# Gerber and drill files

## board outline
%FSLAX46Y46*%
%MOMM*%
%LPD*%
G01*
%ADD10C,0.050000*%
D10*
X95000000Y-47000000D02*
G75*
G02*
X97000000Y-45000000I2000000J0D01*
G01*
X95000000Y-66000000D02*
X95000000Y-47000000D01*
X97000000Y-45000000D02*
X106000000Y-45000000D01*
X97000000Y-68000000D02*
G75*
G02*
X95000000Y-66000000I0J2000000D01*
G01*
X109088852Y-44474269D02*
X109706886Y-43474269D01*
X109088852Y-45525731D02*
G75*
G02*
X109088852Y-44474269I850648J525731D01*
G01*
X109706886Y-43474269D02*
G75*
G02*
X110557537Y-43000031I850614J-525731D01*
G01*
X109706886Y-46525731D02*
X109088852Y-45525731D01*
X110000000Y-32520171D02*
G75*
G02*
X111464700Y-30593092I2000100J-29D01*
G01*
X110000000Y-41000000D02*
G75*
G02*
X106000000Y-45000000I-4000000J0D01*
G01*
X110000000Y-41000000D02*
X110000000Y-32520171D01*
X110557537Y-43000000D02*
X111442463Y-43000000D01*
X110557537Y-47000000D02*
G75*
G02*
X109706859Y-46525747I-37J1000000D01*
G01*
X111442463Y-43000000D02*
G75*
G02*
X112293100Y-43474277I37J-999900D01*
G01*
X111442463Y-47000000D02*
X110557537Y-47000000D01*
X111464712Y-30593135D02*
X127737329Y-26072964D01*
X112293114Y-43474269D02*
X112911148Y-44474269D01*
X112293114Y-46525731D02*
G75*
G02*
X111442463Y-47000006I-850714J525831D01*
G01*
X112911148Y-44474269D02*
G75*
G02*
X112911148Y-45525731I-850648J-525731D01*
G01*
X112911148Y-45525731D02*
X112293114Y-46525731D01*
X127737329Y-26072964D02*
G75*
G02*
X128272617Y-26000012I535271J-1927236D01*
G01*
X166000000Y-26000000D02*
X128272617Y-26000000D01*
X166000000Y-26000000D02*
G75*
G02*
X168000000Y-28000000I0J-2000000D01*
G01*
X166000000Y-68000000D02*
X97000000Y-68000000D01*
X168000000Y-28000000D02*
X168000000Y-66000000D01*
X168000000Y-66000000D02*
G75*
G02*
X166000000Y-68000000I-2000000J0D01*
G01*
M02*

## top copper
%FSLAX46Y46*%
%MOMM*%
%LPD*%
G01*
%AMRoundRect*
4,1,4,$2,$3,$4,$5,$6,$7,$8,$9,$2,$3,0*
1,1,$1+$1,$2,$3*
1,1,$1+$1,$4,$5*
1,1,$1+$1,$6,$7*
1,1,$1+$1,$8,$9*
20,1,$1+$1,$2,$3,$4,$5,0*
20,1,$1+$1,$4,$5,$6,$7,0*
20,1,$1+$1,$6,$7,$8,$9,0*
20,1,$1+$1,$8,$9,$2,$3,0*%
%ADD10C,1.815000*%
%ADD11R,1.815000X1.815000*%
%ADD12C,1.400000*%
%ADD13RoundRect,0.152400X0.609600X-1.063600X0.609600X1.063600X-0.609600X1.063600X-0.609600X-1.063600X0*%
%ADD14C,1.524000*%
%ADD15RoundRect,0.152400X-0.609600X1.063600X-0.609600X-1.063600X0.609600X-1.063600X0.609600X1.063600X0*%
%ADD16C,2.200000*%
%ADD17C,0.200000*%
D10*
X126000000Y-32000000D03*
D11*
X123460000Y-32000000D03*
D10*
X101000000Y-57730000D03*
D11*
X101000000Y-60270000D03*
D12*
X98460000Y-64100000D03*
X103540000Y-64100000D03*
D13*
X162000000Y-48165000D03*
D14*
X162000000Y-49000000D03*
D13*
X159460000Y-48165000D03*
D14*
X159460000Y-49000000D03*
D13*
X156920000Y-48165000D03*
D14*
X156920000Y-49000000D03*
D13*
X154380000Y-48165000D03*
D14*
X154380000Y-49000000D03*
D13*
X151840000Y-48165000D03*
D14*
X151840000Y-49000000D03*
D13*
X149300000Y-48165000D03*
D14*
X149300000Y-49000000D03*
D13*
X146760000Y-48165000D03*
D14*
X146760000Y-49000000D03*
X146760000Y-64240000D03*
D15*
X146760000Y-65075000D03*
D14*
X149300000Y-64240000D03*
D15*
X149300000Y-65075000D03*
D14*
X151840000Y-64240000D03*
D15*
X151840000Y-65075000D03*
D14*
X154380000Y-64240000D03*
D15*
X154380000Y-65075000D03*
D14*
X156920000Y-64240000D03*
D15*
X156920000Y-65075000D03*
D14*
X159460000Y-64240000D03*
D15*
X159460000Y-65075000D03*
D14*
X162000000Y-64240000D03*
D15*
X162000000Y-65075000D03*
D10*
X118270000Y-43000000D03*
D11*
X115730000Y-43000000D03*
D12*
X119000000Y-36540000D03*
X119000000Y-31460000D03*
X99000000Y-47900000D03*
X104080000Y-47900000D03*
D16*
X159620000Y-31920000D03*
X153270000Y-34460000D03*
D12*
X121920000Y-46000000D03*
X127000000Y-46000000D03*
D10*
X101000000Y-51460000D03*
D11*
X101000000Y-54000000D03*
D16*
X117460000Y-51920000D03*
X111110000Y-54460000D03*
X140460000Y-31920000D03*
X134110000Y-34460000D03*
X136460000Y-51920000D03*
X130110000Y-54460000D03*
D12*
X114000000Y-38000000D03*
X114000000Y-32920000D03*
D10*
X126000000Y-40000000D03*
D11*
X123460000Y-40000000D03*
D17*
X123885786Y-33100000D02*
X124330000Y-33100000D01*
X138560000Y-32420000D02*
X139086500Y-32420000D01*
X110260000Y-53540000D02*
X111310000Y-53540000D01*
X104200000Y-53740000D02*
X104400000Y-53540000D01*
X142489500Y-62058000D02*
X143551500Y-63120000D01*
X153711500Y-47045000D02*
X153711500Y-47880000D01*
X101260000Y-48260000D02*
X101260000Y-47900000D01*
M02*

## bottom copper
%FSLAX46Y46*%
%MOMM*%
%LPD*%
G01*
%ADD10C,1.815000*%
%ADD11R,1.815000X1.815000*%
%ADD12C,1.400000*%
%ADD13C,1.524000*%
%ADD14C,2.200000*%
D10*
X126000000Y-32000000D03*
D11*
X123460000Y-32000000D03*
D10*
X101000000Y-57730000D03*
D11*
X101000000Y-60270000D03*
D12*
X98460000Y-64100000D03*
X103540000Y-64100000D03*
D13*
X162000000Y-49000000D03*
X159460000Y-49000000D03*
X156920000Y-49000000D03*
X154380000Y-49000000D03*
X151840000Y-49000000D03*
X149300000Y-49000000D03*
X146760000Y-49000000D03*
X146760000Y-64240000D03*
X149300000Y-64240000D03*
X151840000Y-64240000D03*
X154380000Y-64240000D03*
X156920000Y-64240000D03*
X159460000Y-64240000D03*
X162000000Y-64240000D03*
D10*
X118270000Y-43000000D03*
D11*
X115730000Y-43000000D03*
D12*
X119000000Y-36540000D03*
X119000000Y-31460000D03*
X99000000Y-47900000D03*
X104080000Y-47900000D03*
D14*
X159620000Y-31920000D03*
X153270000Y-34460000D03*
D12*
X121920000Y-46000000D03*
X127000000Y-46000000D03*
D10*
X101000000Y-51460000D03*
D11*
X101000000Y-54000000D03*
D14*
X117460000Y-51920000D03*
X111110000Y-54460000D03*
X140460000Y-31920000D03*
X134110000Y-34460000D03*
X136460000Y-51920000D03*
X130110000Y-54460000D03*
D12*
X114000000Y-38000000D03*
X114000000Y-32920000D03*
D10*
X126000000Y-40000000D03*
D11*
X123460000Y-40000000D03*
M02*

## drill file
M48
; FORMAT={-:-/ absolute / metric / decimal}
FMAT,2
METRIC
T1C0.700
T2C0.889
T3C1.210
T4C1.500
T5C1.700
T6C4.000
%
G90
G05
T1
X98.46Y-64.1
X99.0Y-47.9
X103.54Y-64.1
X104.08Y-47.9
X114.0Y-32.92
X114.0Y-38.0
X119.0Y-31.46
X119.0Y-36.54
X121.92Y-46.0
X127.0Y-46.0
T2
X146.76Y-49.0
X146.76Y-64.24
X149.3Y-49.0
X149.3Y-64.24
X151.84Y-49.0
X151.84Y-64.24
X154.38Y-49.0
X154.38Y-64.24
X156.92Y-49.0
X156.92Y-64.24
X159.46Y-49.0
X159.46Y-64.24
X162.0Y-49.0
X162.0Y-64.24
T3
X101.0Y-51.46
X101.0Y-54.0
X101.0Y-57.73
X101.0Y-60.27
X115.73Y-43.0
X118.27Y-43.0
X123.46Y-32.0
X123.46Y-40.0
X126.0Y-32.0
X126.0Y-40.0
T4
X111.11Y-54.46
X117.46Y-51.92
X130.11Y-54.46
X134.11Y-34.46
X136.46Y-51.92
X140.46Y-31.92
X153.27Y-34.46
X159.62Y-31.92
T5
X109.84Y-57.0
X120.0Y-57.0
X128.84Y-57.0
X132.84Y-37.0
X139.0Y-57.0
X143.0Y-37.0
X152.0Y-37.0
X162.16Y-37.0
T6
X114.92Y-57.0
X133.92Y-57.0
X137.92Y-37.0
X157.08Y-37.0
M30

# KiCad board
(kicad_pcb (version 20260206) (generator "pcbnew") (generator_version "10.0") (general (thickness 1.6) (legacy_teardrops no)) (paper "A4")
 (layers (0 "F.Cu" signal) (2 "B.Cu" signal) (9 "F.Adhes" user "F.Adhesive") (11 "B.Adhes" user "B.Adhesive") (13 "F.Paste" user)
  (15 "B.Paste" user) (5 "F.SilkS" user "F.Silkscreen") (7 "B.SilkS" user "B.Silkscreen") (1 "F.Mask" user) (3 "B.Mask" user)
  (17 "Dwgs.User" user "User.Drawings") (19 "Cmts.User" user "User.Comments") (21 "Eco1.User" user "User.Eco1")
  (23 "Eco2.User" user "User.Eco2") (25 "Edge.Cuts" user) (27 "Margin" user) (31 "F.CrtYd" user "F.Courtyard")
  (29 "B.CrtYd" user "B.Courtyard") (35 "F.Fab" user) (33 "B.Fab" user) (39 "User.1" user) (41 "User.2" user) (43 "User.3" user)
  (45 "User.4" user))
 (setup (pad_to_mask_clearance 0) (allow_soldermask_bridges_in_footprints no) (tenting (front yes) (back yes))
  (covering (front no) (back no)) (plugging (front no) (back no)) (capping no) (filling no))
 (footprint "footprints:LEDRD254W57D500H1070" (layer "F.Cu") (at 124.73 32)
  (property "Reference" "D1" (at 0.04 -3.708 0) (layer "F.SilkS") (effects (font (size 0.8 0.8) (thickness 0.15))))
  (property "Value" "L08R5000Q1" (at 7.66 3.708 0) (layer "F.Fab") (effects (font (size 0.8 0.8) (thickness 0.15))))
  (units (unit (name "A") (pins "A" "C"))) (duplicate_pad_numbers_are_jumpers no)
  (pad "A" thru_hole circle (at 1.27 0) (size 1.815 1.815) (drill 1.21) (layers "*.Cu" "*.Mask") (remove_unused_layers no)
   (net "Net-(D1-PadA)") (solder_mask_margin 0.102))
  (pad "C" thru_hole rect (at -1.27 0) (size 1.815 1.815) (drill 1.21) (layers "*.Cu" "*.Mask") (remove_unused_layers no) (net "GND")
   (solder_mask_margin 0.102)))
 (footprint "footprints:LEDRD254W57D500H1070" (layer "F.Cu") (at 101 59 90)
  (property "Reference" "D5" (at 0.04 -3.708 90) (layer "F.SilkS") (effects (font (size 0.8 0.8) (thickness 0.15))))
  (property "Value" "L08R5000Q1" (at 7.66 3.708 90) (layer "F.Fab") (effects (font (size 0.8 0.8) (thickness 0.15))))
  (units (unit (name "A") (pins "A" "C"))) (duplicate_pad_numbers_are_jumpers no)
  (pad "A" thru_hole circle (at 1.27 0 90) (size 1.815 1.815) (drill 1.21) (layers "*.Cu" "*.Mask") (remove_unused_layers no)
   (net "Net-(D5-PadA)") (solder_mask_margin 0.102))
  (pad "C" thru_hole rect (at -1.27 0 90) (size 1.815 1.815) (drill 1.21) (layers "*.Cu" "*.Mask") (remove_unused_layers no) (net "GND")
   (solder_mask_margin 0.102)))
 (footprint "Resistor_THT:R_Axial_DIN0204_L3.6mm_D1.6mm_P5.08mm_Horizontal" (layer "F.Cu") (at 98.46 64.1)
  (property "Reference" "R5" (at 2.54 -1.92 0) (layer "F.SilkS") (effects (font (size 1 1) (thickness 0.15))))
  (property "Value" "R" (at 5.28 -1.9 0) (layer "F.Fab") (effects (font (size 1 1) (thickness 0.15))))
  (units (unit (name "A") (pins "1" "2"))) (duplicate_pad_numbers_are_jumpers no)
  (pad "1" thru_hole circle (at 0 0) (size 1.4 1.4) (drill 0.7) (layers "*.Cu" "*.Mask") (remove_unused_layers no) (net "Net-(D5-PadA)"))
  (pad "2" thru_hole circle (at 5.08 0) (size 1.4 1.4) (drill 0.7) (layers "*.Cu" "*.Mask") (remove_unused_layers no) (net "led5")))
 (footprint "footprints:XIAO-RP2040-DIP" (layer "F.Cu") (at 154.38 56.62)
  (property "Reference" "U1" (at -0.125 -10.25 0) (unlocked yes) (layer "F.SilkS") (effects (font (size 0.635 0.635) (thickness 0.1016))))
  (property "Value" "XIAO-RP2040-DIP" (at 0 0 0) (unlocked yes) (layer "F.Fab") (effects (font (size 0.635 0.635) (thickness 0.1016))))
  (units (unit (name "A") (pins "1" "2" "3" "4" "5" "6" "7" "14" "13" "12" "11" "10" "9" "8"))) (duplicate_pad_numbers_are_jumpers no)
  (pad "1" smd roundrect (at 7.62 -8.455 90) (size 2.432 1.524) (layers "F.Cu" "F.Mask") (roundrect_rratio 0.1) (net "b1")
   (thermal_bridge_angle 45))
  (pad "1" thru_hole circle (at 7.62 -7.62 90) (size 1.524 1.524) (drill 0.889) (layers "*.Cu" "*.Mask") (remove_unused_layers no)
   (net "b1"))
  (pad "2" smd roundrect (at 5.08 -8.455 90) (size 2.432 1.524) (layers "F.Cu" "F.Mask") (roundrect_rratio 0.1) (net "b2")
   (thermal_bridge_angle 45))
  (pad "2" thru_hole circle (at 5.08 -7.62 90) (size 1.524 1.524) (drill 0.889) (layers "*.Cu" "*.Mask") (remove_unused_layers no)
   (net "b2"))
  (pad "3" smd roundrect (at 2.54 -8.455 90) (size 2.432 1.524) (layers "F.Cu" "F.Mask") (roundrect_rratio 0.1) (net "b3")
   (thermal_bridge_angle 45))
  (pad "3" thru_hole circle (at 2.54 -7.62 90) (size 1.524 1.524) (drill 0.889) (layers "*.Cu" "*.Mask") (remove_unused_layers no)
   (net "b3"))
  (pad "4" smd roundrect (at 0 -8.455 90) (size 2.432 1.524) (layers "F.Cu" "F.Mask") (roundrect_rratio 0.1) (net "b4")
   (thermal_bridge_angle 45))
  (pad "4" thru_hole circle (at 0 -7.62 90) (size 1.524 1.524) (drill 0.889) (layers "*.Cu" "*.Mask") (remove_unused_layers no) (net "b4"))
  (pad "5" smd roundrect (at -2.54 -8.455 90) (size 2.432 1.524) (layers "F.Cu" "F.Mask") (roundrect_rratio 0.1) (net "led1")
   (thermal_bridge_angle 45))
  (pad "5" thru_hole circle (at -2.54 -7.62 90) (size 1.524 1.524) (drill 0.889) (layers "*.Cu" "*.Mask") (remove_unused_layers no)
   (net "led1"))
  (pad "6" smd roundrect (at -5.08 -8.455 90) (size 2.432 1.524) (layers "F.Cu" "F.Mask") (roundrect_rratio 0.1) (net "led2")
   (thermal_bridge_angle 45))
  (pad "6" thru_hole circle (at -5.08 -7.62 90) (size 1.524 1.524) (drill 0.889) (layers "*.Cu" "*.Mask") (remove_unused_layers no)
   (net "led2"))
  (pad "7" smd roundrect (at -7.62 -8.455 90) (size 2.432 1.524) (layers "F.Cu" "F.Mask") (roundrect_rratio 0.1) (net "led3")
   (thermal_bridge_angle 45))
  (pad "7" thru_hole circle (at -7.62 -7.62 90) (size 1.524 1.524) (drill 0.889) (layers "*.Cu" "*.Mask") (remove_unused_layers no)
   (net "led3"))
  (pad "8" thru_hole circle (at -7.62 7.62 270) (size 1.524 1.524) (drill 0.889) (layers "*.Cu" "*.Mask") (remove_unused_layers no)
   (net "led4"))
  (pad "8" smd roundrect (at -7.62 8.455 270) (size 2.432 1.524) (layers "F.Cu" "F.Mask") (roundrect_rratio 0.1) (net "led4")
   (thermal_bridge_angle 45))
  (pad "9" thru_hole circle (at -5.08 7.62 270) (size 1.524 1.524) (drill 0.889) (layers "*.Cu" "*.Mask") (remove_unused_layers no)
   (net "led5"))
  (pad "9" smd roundrect (at -5.08 8.455 270) (size 2.432 1.524) (layers "F.Cu" "F.Mask") (roundrect_rratio 0.1) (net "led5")
   (thermal_bridge_angle 45))
  (pad "10" thru_hole circle (at -2.54 7.62 270) (size 1.524 1.524) (drill 0.889) (layers "*.Cu" "*.Mask") (remove_unused_layers no)
   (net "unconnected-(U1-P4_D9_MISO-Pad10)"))
  (pad "10" smd roundrect (at -2.54 8.455 270) (size 2.432 1.524) (layers "F.Cu" "F.Mask") (roundrect_rratio 0.1)
   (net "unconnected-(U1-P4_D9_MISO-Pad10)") (thermal_bridge_angle 45))
  (pad "11" thru_hole circle (at 0 7.62 270) (size 1.524 1.524) (drill 0.889) (layers "*.Cu" "*.Mask") (remove_unused_layers no)
   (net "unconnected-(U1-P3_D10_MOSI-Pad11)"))
  (pad "11" smd roundrect (at 0 8.455 270) (size 2.432 1.524) (layers "F.Cu" "F.Mask") (roundrect_rratio 0.1)
   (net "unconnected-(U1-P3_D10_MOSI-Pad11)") (thermal_bridge_angle 45))
  (pad "12" thru_hole circle (at 2.54 7.62 270) (size 1.524 1.524) (drill 0.889) (layers "*.Cu" "*.Mask") (remove_unused_layers no)
   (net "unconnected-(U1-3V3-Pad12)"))
  (pad "12" smd roundrect (at 2.54 8.455 270) (size 2.432 1.524) (layers "F.Cu" "F.Mask") (roundrect_rratio 0.1)
   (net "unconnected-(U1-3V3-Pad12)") (thermal_bridge_angle 45))
  (pad "13" thru_hole circle (at 5.08 7.62 270) (size 1.524 1.524) (drill 0.889) (layers "*.Cu" "*.Mask") (remove_unused_layers no)
   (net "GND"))
  (pad "13" smd roundrect (at 5.08 8.455 270) (size 2.432 1.524) (layers "F.Cu" "F.Mask") (roundrect_rratio 0.1) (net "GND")
   (thermal_bridge_angle 45))
  (pad "14" thru_hole circle (at 7.62 7.62 270) (size 1.524 1.524) (drill 0.889) (layers "*.Cu" "*.Mask") (remove_unused_layers no)
   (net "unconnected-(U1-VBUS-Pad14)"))
  (pad "14" smd roundrect (at 7.62 8.455 270) (size 2.432 1.524) (layers "F.Cu" "F.Mask") (roundrect_rratio 0.1)
   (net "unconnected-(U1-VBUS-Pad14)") (thermal_bridge_angle 45)))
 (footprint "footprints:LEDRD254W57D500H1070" (layer "F.Cu") (at 117 43)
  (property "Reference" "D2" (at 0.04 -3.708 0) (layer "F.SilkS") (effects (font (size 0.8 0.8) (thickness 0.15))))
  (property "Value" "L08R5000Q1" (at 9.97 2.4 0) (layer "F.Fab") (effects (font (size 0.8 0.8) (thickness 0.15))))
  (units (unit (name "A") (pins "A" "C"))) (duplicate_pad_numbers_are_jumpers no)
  (pad "A" thru_hole circle (at 1.27 0) (size 1.815 1.815) (drill 1.21) (layers "*.Cu" "*.Mask") (remove_unused_layers no)
   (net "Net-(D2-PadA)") (solder_mask_margin 0.102))
  (pad "C" thru_hole rect (at -1.27 0) (size 1.815 1.815) (drill 1.21) (layers "*.Cu" "*.Mask") (remove_unused_layers no) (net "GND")
   (solder_mask_margin 0.102)))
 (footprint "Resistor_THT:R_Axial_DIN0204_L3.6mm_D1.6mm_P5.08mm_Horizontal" (layer "F.Cu") (at 119 36.54 90)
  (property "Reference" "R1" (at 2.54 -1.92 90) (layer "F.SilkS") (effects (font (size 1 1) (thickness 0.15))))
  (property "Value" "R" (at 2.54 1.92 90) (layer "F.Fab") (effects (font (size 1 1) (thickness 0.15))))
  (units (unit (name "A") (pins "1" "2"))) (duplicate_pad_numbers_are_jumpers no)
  (pad "1" thru_hole circle (at 0 0 90) (size 1.4 1.4) (drill 0.7) (layers "*.Cu" "*.Mask") (remove_unused_layers no) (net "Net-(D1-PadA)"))
  (pad "2" thru_hole circle (at 5.08 0 90) (size 1.4 1.4) (drill 0.7) (layers "*.Cu" "*.Mask") (remove_unused_layers no) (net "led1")))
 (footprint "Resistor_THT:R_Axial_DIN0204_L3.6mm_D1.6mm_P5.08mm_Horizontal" (layer "F.Cu") (at 99 47.9)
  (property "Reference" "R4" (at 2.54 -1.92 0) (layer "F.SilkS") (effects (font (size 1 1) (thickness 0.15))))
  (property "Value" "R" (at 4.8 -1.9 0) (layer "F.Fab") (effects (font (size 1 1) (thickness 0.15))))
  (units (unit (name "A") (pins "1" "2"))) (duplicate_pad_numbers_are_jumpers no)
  (pad "1" thru_hole circle (at 0 0) (size 1.4 1.4) (drill 0.7) (layers "*.Cu" "*.Mask") (remove_unused_layers no) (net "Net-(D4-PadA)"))
  (pad "2" thru_hole circle (at 5.08 0) (size 1.4 1.4) (drill 0.7) (layers "*.Cu" "*.Mask") (remove_unused_layers no) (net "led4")))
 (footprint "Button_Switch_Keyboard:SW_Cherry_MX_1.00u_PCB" (layer "F.Cu") (at 159.62 31.92)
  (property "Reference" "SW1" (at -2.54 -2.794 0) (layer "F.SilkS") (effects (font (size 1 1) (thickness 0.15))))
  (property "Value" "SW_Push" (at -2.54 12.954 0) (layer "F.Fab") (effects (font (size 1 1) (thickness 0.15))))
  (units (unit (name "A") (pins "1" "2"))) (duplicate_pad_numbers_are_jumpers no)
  (pad "" np_thru_hole circle (at -7.62 5.08) (size 1.7 1.7) (drill 1.7) (layers "*.Cu" "*.Mask"))
  (pad "" np_thru_hole circle (at -2.54 5.08) (size 4 4) (drill 4) (layers "*.Cu" "*.Mask"))
  (pad "" np_thru_hole circle (at 2.54 5.08) (size 1.7 1.7) (drill 1.7) (layers "*.Cu" "*.Mask"))
  (pad "1" thru_hole circle (at 0 0) (size 2.2 2.2) (drill 1.5) (layers "*.Cu" "*.Mask") (remove_unused_layers no) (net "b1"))
  (pad "2" thru_hole circle (at -6.35 2.54) (size 2.2 2.2) (drill 1.5) (layers "*.Cu" "*.Mask") (remove_unused_layers no) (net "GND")))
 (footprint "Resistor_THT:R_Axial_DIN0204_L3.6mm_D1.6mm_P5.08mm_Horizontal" (layer "F.Cu") (at 121.92 46)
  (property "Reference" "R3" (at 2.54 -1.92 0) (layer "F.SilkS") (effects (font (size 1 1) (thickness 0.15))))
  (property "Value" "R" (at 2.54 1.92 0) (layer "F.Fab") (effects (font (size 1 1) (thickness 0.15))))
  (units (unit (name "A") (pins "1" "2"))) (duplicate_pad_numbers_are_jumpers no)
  (pad "1" thru_hole circle (at 0 0) (size 1.4 1.4) (drill 0.7) (layers "*.Cu" "*.Mask") (remove_unused_layers no) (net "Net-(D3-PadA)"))
  (pad "2" thru_hole circle (at 5.08 0) (size 1.4 1.4) (drill 0.7) (layers "*.Cu" "*.Mask") (remove_unused_layers no) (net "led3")))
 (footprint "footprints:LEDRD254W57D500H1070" (layer "F.Cu") (at 101 52.73 90)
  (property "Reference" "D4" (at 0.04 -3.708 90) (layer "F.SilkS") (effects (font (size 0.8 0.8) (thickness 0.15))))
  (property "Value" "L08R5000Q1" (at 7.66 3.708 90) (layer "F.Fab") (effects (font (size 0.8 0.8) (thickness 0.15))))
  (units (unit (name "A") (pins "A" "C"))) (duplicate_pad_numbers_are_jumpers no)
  (pad "A" thru_hole circle (at 1.27 0 90) (size 1.815 1.815) (drill 1.21) (layers "*.Cu" "*.Mask") (remove_unused_layers no)
   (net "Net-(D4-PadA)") (solder_mask_margin 0.102))
  (pad "C" thru_hole rect (at -1.27 0 90) (size 1.815 1.815) (drill 1.21) (layers "*.Cu" "*.Mask") (remove_unused_layers no) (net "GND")
   (solder_mask_margin 0.102)))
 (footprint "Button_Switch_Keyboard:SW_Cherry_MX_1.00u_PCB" (layer "F.Cu") (at 117.46 51.92)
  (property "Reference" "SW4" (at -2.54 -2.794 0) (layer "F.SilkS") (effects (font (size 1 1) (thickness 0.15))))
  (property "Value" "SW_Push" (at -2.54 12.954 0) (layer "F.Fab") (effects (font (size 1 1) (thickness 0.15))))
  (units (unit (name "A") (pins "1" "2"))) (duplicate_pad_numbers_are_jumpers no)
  (pad "" np_thru_hole circle (at -7.62 5.08) (size 1.7 1.7) (drill 1.7) (layers "*.Cu" "*.Mask"))
  (pad "" np_thru_hole circle (at -2.54 5.08) (size 4 4) (drill 4) (layers "*.Cu" "*.Mask"))
  (pad "" np_thru_hole circle (at 2.54 5.08) (size 1.7 1.7) (drill 1.7) (layers "*.Cu" "*.Mask"))
  (pad "1" thru_hole circle (at 0 0) (size 2.2 2.2) (drill 1.5) (layers "*.Cu" "*.Mask") (remove_unused_layers no) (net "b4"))
  (pad "2" thru_hole circle (at -6.35 2.54) (size 2.2 2.2) (drill 1.5) (layers "*.Cu" "*.Mask") (remove_unused_layers no) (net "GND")))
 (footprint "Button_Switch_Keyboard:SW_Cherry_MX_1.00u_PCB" (layer "F.Cu") (at 140.46 31.92)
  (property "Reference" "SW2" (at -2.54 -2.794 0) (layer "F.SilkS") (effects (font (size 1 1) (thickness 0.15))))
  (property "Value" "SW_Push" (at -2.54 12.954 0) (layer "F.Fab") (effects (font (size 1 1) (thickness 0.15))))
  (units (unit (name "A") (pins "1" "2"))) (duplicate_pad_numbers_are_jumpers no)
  (pad "" np_thru_hole circle (at -7.62 5.08) (size 1.7 1.7) (drill 1.7) (layers "*.Cu" "*.Mask"))
  (pad "" np_thru_hole circle (at -2.54 5.08) (size 4 4) (drill 4) (layers "*.Cu" "*.Mask"))
  (pad "" np_thru_hole circle (at 2.54 5.08) (size 1.7 1.7) (drill 1.7) (layers "*.Cu" "*.Mask"))
  (pad "1" thru_hole circle (at 0 0) (size 2.2 2.2) (drill 1.5) (layers "*.Cu" "*.Mask") (remove_unused_layers no) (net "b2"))
  (pad "2" thru_hole circle (at -6.35 2.54) (size 2.2 2.2) (drill 1.5) (layers "*.Cu" "*.Mask") (remove_unused_layers no) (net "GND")))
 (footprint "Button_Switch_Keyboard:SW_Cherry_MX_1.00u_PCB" (layer "F.Cu") (at 136.46 51.92)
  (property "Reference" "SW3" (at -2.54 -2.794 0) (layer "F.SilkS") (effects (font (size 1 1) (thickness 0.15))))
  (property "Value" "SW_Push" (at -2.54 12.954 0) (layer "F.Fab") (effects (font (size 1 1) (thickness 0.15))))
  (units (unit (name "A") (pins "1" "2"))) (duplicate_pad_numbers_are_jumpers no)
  (pad "" np_thru_hole circle (at -7.62 5.08) (size 1.7 1.7) (drill 1.7) (layers "*.Cu" "*.Mask"))
  (pad "" np_thru_hole circle (at -2.54 5.08) (size 4 4) (drill 4) (layers "*.Cu" "*.Mask"))
  (pad "" np_thru_hole circle (at 2.54 5.08) (size 1.7 1.7) (drill 1.7) (layers "*.Cu" "*.Mask"))
  (pad "1" thru_hole circle (at 0 0) (size 2.2 2.2) (drill 1.5) (layers "*.Cu" "*.Mask") (remove_unused_layers no) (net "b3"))
  (pad "2" thru_hole circle (at -6.35 2.54) (size 2.2 2.2) (drill 1.5) (layers "*.Cu" "*.Mask") (remove_unused_layers no) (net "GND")))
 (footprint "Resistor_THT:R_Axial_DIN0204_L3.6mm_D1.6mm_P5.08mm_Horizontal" (layer "F.Cu") (at 114 38 90)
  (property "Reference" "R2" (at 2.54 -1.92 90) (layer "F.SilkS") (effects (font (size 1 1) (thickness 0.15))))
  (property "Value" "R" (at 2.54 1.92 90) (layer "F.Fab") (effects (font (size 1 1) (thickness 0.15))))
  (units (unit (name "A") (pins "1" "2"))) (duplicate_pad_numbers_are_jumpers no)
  (pad "1" thru_hole circle (at 0 0 90) (size 1.4 1.4) (drill 0.7) (layers "*.Cu" "*.Mask") (remove_unused_layers no) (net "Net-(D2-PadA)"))
  (pad "2" thru_hole circle (at 5.08 0 90) (size 1.4 1.4) (drill 0.7) (layers "*.Cu" "*.Mask") (remove_unused_layers no) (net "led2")))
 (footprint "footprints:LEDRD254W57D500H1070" (layer "F.Cu") (at 124.73 40)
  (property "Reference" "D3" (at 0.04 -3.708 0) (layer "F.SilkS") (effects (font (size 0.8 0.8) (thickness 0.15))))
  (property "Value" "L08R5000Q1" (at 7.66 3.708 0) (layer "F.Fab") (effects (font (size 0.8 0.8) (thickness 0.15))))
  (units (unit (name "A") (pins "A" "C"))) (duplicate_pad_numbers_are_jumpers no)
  (pad "A" thru_hole circle (at 1.27 0) (size 1.815 1.815) (drill 1.21) (layers "*.Cu" "*.Mask") (remove_unused_layers no)
   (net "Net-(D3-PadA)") (solder_mask_margin 0.102))
  (pad "C" thru_hole rect (at -1.27 0) (size 1.815 1.815) (drill 1.21) (layers "*.Cu" "*.Mask") (remove_unused_layers no) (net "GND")
   (solder_mask_margin 0.102)))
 (gr_arc (start 95 47) (mid 95.585786 45.585786) (end 97 45) (stroke (width 0.05) (type default)) (layer "Edge.Cuts"))
 (gr_line (start 95 66) (end 95 47) (stroke (width 0.05) (type default)) (layer "Edge.Cuts"))
 (gr_line (start 97 45) (end 106 45) (stroke (width 0.05) (type default)) (layer "Edge.Cuts"))
 (gr_arc (start 97 68) (mid 95.585786 67.414214) (end 95 66) (stroke (width 0.05) (type default)) (layer "Edge.Cuts"))
 (gr_line (start 109.088852 44.474269) (end 109.706886 43.474269) (stroke (width 0.05) (type default)) (layer "Edge.Cuts"))
 (gr_arc (start 109.088852 45.525731) (mid 108.939503 45) (end 109.088852 44.474269) (stroke (width 0.05) (type default))
  (layer "Edge.Cuts"))
 (gr_arc (start 109.706886 43.474269) (mid 110.070572 43.126578) (end 110.557537 43) (stroke (width 0.05) (type default))
  (layer "Edge.Cuts"))
 (gr_line (start 109.706886 46.525731) (end 109.088852 45.525731) (stroke (width 0.05) (type default)) (layer "Edge.Cuts"))
 (gr_arc (start 110 32.520171) (mid 110.407752 31.309932) (end 111.464712 30.593135) (stroke (width 0.05) (type default))
  (layer "Edge.Cuts"))
 (gr_arc (start 110 41) (mid 108.828427 43.828427) (end 106 45) (stroke (width 0.05) (type default)) (layer "Edge.Cuts"))
 (gr_line (start 110 41) (end 110 32.520171) (stroke (width 0.05) (type default)) (layer "Edge.Cuts"))
 (gr_line (start 110.557537 43) (end 111.442463 43) (stroke (width 0.05) (type default)) (layer "Edge.Cuts"))
 (gr_arc (start 110.557537 47) (mid 110.070572 46.873422) (end 109.706886 46.525731) (stroke (width 0.05) (type default))
  (layer "Edge.Cuts"))
 (gr_arc (start 111.442463 43) (mid 111.92944 43.126565) (end 112.293114 43.474269) (stroke (width 0.05) (type default)) (layer "Edge.Cuts"))
 (gr_line (start 111.442463 47) (end 110.557537 47) (stroke (width 0.05) (type default)) (layer "Edge.Cuts"))
 (gr_line (start 111.464712 30.593135) (end 127.737329 26.072964) (stroke (width 0.05) (type default)) (layer "Edge.Cuts"))
 (gr_line (start 112.293114 43.474269) (end 112.911148 44.474269) (stroke (width 0.05) (type default)) (layer "Edge.Cuts"))
 (gr_arc (start 112.293114 46.525731) (mid 111.929425 46.873408) (end 111.442463 47) (stroke (width 0.05) (type default))
  (layer "Edge.Cuts"))
 (gr_arc (start 112.911148 44.474269) (mid 113.060497 45) (end 112.911148 45.525731) (stroke (width 0.05) (type default))
  (layer "Edge.Cuts"))
 (gr_line (start 112.911148 45.525731) (end 112.293114 46.525731) (stroke (width 0.05) (type default)) (layer "Edge.Cuts"))
 (gr_arc (start 127.737329 26.072964) (mid 128.002498 26.018327) (end 128.272617 26) (stroke (width 0.05) (type default))
  (layer "Edge.Cuts"))
 (gr_line (start 166 26) (end 128.272617 26) (stroke (width 0.05) (type default)) (layer "Edge.Cuts"))
 (gr_arc (start 166 26) (mid 167.414214 26.585786) (end 168 28) (stroke (width 0.05) (type default)) (layer "Edge.Cuts"))
 (gr_line (start 166 68) (end 97 68) (stroke (width 0.05) (type default)) (layer "Edge.Cuts"))
 (gr_line (start 168 28) (end 168 66) (stroke (width 0.05) (type default)) (layer "Edge.Cuts"))
 (gr_arc (start 168 66) (mid 167.414214 67.414214) (end 166 68) (stroke (width 0.05) (type default)) (layer "Edge.Cuts"))
 (segment (start 123.885786 33.1) (end 124.33 33.1) (width 0.2) (layer "F.Cu") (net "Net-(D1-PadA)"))
 (segment (start 138.56 32.42) (end 139.0865 32.42) (width 0.2) (layer "F.Cu") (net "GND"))
 (segment (start 110.26 53.54) (end 111.31 53.54) (width 0.2) (layer "F.Cu") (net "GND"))
 (segment (start 104.2 53.74) (end 104.4 53.54) (width 0.2) (layer "F.Cu") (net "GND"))
 (segment (start 142.4895 62.058) (end 143.5515 63.12) (width 0.2) (layer "F.Cu") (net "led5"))
 (segment (start 153.7115 47.045) (end 153.7115 47.88) (width 0.2) (layer "F.Cu") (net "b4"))
 (segment (start 101.26 48.26) (end 101.26 47.9) (width 0.2) (layer "F.Cu") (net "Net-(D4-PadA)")))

